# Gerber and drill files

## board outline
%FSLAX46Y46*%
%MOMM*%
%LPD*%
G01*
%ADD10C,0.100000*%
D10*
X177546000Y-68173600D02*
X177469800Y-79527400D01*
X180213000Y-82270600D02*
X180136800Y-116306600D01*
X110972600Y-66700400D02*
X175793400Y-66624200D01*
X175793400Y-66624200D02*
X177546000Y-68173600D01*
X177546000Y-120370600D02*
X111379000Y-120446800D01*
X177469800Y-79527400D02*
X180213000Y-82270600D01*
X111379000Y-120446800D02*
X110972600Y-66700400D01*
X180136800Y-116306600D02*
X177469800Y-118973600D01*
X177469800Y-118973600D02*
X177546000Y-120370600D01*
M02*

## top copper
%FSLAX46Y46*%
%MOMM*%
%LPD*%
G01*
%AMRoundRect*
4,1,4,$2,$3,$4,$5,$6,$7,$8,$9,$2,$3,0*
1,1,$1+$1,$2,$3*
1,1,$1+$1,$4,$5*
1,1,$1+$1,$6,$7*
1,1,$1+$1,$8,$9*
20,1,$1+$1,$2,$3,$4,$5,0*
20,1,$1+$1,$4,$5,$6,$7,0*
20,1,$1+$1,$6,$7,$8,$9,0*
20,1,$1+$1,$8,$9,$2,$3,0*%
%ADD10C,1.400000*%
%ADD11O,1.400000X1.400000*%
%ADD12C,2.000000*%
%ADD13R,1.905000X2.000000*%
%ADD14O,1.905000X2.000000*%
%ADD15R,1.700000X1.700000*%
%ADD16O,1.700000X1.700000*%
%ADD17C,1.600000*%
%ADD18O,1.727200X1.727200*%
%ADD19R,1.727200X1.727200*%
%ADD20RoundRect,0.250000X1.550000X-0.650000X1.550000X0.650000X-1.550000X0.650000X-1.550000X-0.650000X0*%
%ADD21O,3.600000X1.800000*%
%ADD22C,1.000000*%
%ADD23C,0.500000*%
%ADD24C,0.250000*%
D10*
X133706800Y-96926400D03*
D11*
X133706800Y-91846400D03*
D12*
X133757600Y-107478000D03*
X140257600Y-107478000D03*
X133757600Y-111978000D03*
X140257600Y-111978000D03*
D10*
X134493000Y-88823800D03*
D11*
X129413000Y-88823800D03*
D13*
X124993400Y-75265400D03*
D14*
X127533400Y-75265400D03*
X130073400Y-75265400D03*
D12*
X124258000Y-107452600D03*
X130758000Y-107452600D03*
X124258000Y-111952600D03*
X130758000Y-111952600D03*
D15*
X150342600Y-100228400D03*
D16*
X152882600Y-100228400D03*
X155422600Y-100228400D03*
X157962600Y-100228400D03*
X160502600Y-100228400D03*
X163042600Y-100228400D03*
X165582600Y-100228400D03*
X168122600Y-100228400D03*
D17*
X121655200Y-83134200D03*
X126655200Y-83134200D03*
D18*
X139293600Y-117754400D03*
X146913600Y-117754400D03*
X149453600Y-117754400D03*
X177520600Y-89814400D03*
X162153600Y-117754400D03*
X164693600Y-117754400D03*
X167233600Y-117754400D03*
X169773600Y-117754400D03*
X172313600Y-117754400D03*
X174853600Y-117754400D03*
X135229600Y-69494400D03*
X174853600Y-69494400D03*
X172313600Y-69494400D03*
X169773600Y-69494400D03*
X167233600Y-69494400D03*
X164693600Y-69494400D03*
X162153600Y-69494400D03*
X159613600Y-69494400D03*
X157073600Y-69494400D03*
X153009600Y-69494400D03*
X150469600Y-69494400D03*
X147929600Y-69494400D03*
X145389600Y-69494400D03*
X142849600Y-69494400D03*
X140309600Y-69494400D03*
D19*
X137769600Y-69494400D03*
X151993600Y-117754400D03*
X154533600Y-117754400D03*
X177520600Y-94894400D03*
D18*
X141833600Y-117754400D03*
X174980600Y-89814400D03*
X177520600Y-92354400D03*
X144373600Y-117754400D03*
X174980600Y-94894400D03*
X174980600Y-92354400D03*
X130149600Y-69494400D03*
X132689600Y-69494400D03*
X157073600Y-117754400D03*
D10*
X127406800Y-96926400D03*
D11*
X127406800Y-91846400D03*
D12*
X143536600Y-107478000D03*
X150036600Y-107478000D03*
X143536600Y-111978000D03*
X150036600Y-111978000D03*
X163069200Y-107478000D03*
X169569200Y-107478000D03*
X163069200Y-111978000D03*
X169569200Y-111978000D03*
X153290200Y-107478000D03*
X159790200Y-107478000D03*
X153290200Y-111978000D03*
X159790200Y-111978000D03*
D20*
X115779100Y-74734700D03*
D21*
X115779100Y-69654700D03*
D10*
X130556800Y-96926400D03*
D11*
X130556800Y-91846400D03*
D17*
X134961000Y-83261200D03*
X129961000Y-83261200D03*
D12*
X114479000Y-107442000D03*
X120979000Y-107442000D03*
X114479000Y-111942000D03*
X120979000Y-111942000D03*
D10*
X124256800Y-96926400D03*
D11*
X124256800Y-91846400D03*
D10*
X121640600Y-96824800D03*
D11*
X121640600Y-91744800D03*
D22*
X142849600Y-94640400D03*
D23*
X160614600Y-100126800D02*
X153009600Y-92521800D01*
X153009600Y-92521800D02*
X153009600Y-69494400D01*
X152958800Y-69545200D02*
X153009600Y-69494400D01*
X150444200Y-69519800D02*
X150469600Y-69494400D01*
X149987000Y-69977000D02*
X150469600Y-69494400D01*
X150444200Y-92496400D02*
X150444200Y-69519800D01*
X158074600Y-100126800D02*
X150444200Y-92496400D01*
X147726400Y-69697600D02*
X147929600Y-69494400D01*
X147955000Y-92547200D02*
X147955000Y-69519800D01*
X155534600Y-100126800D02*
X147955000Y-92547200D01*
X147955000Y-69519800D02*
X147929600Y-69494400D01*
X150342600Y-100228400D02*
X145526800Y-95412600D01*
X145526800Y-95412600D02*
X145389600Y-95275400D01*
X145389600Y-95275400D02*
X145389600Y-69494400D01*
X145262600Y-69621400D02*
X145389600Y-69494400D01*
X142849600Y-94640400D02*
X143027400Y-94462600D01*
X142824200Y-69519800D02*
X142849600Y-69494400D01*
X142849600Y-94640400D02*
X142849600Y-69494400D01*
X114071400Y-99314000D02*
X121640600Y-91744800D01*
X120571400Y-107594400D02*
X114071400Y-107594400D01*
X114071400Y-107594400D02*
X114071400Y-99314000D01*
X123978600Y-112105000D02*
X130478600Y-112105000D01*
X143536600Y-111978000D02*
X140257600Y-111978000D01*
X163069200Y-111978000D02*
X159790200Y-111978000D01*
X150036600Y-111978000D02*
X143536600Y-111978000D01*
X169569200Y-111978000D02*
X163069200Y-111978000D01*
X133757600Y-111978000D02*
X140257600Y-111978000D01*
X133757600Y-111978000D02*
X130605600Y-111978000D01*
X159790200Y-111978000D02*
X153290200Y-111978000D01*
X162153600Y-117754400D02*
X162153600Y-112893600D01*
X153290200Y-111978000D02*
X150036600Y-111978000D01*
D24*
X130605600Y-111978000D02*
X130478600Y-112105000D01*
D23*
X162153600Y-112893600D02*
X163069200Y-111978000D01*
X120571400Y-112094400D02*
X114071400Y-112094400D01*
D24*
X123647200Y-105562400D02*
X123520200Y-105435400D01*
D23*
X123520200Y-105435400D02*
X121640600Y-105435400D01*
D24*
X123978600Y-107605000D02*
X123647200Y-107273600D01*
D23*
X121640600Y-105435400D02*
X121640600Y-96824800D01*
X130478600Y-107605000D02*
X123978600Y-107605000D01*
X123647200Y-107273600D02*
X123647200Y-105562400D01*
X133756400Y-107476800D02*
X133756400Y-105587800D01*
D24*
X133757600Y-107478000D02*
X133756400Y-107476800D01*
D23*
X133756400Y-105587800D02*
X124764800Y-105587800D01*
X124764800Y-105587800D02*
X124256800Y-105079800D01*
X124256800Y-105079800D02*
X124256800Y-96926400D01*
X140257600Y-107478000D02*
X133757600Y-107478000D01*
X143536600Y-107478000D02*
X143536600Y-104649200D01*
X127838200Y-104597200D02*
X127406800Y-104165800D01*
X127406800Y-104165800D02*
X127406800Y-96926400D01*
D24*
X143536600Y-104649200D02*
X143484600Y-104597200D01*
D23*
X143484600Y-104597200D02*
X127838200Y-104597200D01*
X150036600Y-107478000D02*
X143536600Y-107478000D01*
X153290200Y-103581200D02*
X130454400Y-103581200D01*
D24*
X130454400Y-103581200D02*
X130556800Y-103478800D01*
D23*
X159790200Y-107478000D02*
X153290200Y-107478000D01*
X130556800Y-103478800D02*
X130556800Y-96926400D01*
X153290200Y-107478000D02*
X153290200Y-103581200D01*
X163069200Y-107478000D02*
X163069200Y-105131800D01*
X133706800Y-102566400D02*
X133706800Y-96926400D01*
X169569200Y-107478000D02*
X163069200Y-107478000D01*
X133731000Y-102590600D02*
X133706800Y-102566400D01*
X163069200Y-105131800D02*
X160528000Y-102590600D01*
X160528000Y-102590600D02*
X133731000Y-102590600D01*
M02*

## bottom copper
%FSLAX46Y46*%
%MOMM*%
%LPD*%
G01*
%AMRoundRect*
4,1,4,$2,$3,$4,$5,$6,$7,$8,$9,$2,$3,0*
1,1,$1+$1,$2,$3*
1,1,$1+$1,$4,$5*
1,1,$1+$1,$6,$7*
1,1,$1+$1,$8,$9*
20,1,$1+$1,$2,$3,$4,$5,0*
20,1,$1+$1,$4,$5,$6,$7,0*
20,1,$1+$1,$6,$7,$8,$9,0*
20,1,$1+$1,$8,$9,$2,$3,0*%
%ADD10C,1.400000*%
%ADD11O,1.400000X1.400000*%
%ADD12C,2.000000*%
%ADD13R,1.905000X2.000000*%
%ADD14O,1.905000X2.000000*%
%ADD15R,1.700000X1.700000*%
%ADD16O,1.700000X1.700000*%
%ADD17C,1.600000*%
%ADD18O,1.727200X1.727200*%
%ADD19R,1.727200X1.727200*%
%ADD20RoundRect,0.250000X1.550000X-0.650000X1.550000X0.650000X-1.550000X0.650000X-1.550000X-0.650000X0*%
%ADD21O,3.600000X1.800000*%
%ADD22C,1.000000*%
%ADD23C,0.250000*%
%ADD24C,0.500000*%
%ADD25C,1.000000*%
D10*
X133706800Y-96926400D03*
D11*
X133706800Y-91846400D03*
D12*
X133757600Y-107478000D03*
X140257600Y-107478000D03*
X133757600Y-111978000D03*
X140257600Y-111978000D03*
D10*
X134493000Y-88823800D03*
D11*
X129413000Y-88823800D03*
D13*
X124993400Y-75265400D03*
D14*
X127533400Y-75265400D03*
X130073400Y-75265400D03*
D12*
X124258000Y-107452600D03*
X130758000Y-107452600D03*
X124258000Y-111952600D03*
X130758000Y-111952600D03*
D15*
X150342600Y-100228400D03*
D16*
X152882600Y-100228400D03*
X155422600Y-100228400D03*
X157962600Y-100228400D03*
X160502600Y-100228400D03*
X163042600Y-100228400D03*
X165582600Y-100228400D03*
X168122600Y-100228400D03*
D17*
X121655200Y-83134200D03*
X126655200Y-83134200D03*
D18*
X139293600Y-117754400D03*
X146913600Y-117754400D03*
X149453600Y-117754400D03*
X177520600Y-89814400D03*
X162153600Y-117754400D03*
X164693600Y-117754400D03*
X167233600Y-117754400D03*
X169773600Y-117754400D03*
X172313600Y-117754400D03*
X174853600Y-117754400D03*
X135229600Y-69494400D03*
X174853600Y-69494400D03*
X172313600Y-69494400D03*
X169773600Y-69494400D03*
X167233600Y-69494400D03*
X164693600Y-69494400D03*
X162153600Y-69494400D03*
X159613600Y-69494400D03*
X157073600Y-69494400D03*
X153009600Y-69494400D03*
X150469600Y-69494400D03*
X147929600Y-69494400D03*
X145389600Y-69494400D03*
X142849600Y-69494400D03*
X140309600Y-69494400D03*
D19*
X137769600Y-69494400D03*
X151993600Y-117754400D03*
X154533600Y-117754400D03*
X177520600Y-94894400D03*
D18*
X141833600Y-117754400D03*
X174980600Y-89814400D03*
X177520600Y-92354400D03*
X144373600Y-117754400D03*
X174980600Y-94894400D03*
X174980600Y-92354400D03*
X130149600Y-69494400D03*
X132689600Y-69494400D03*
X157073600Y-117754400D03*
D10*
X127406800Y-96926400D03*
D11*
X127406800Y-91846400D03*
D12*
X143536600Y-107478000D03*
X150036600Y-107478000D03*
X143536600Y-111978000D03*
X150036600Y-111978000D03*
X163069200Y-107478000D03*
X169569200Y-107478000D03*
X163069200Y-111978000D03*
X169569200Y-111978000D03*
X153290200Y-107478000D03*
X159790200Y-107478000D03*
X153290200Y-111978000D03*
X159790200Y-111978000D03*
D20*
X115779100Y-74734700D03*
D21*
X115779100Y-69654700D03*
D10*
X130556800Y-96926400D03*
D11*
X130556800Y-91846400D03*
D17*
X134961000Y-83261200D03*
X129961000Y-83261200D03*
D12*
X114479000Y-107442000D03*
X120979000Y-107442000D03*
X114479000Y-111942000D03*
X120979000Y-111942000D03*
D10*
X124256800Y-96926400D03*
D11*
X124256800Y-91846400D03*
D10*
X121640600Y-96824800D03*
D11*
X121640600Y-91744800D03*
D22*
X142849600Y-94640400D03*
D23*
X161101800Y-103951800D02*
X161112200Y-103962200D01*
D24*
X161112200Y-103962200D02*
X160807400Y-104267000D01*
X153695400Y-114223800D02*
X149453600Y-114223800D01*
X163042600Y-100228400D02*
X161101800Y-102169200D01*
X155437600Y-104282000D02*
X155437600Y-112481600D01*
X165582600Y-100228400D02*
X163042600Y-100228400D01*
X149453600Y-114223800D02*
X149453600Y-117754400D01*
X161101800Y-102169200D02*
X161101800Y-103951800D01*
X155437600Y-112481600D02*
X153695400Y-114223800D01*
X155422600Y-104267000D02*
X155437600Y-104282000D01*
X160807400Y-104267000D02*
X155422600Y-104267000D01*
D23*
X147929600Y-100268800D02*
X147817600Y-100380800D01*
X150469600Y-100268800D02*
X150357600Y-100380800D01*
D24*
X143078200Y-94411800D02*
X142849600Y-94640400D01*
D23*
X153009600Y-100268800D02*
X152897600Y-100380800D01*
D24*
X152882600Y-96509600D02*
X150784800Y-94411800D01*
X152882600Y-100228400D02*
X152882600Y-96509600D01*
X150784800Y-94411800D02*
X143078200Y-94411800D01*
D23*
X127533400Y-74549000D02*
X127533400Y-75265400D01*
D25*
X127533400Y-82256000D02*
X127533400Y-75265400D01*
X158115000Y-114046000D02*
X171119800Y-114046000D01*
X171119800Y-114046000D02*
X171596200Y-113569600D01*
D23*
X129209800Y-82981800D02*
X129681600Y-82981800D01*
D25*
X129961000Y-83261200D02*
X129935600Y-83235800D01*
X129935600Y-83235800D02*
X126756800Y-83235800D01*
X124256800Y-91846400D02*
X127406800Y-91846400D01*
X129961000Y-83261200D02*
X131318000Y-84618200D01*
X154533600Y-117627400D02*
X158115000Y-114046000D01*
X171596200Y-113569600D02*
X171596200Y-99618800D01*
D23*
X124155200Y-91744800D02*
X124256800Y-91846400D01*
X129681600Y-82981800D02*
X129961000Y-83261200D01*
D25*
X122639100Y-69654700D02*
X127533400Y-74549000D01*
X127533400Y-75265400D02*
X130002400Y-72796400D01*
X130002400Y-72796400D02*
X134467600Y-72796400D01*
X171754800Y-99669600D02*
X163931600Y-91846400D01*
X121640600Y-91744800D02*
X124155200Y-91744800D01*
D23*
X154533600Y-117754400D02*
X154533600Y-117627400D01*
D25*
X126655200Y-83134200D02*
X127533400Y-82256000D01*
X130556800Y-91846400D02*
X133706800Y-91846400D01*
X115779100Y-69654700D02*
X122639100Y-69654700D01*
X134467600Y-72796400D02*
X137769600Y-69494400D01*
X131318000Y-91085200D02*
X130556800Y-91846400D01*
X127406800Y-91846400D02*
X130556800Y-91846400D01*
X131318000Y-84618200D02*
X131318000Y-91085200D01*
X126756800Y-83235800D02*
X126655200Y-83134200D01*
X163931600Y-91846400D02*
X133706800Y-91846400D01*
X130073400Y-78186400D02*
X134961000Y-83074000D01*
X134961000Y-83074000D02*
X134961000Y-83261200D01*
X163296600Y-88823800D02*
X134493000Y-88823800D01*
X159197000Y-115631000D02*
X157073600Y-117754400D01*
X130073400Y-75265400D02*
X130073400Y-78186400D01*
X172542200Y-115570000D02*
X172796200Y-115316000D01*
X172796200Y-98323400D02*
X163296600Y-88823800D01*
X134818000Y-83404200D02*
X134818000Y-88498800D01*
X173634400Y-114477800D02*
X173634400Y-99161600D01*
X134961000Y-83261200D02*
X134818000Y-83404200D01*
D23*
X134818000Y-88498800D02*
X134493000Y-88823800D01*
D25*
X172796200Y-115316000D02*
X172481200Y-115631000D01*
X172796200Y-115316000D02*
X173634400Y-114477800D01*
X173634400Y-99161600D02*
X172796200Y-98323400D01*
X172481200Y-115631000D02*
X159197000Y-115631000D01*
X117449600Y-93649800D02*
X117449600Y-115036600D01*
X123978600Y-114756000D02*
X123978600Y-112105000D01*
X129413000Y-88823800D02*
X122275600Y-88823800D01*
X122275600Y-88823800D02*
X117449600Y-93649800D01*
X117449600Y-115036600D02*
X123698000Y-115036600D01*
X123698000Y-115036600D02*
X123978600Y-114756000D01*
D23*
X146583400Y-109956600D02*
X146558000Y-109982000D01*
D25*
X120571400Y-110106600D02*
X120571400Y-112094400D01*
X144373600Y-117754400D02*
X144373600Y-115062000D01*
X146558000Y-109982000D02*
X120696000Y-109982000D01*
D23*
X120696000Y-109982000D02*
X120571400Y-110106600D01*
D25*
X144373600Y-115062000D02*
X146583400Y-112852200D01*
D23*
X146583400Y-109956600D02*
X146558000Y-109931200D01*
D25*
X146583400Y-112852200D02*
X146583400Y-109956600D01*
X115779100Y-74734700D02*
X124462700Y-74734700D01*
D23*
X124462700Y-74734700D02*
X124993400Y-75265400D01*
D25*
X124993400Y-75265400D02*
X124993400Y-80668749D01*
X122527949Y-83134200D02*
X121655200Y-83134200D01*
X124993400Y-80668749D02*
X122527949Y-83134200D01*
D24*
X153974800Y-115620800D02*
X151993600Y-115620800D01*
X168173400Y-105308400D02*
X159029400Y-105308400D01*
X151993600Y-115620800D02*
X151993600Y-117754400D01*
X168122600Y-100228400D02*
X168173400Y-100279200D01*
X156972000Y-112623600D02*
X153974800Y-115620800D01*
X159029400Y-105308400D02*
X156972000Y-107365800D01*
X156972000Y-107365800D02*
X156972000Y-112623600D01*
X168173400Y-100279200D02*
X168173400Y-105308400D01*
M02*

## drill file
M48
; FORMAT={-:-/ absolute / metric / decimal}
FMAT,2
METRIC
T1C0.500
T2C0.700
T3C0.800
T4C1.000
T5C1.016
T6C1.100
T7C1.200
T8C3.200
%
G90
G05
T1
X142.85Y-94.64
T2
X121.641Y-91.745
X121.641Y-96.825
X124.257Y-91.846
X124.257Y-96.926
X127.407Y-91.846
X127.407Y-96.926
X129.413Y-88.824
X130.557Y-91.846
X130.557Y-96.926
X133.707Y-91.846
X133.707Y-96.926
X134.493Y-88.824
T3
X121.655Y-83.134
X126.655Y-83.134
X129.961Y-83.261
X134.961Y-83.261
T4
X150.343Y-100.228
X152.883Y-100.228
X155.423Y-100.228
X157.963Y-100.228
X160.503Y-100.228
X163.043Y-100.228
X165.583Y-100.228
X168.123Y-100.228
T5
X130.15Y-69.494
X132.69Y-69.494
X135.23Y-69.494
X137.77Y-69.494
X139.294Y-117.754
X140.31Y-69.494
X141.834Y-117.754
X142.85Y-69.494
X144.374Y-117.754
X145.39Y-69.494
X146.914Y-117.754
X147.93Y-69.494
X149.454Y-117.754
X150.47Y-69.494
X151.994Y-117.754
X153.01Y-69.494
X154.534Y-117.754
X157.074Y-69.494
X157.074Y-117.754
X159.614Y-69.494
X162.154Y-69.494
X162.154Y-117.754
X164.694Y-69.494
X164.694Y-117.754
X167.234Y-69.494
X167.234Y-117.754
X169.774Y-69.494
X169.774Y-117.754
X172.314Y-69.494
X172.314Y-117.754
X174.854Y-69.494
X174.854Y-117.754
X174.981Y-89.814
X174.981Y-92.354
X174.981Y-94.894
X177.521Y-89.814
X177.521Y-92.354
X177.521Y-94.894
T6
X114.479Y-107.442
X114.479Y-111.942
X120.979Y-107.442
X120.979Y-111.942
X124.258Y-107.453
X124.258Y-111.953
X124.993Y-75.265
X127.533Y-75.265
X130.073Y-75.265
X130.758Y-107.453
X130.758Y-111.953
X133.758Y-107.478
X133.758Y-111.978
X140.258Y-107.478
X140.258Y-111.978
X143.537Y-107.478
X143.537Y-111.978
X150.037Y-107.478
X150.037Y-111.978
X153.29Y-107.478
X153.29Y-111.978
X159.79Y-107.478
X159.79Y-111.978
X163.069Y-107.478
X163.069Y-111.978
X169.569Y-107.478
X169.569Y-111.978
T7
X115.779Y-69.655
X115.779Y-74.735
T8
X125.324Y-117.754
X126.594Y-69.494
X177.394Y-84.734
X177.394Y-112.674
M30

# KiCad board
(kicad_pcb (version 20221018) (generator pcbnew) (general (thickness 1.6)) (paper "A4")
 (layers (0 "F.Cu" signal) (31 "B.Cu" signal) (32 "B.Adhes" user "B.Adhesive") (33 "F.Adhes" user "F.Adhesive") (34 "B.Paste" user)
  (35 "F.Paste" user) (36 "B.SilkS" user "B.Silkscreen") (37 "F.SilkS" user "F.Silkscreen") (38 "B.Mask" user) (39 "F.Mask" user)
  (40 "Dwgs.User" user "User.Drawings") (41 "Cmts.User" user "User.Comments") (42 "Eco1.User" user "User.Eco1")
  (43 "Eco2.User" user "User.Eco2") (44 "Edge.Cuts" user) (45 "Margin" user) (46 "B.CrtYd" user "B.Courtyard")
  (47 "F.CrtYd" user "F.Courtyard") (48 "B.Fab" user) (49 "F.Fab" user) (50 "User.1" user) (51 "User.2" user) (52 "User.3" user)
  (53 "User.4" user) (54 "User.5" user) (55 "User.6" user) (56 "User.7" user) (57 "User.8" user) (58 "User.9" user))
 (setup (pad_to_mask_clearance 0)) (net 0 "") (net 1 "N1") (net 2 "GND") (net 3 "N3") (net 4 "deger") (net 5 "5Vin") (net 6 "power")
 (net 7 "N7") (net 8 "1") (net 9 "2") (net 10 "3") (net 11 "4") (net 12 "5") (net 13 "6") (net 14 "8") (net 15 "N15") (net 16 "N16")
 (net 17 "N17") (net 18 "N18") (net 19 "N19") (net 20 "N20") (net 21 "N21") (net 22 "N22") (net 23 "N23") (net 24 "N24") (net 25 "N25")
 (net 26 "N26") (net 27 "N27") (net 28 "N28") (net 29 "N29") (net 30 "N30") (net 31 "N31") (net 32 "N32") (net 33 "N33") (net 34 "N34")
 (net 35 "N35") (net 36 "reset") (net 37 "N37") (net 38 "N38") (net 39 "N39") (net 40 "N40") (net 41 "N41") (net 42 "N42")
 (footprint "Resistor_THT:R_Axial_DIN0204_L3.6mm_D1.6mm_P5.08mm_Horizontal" (layer "F.Cu") (at 133.7068 96.9264 90)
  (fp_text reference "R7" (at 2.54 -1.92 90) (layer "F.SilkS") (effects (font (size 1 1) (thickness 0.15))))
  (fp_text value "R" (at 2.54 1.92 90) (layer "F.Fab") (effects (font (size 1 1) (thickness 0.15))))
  (pad "1" thru_hole circle (at 0 0 90) (size 1.4 1.4) (drill 0.7) (layers "*.Cu" "*.Mask") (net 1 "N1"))
  (pad "2" thru_hole oval (at 5.08 0 90) (size 1.4 1.4) (drill 0.7) (layers "*.Cu" "*.Mask") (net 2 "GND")))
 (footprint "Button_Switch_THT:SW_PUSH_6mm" (layer "F.Cu") (at 133.7576 107.478)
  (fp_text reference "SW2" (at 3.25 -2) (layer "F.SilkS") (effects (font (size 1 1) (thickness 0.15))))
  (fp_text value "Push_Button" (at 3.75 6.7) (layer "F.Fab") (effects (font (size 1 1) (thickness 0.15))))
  (pad "1" thru_hole circle (at 0 0 90) (size 2 2) (drill 1.1) (layers "*.Cu" "*.Mask") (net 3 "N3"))
  (pad "1" thru_hole circle (at 6.5 0 90) (size 2 2) (drill 1.1) (layers "*.Cu" "*.Mask") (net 3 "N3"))
  (pad "2" thru_hole circle (at 0 4.5 90) (size 2 2) (drill 1.1) (layers "*.Cu" "*.Mask") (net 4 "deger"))
  (pad "2" thru_hole circle (at 6.5 4.5 90) (size 2 2) (drill 1.1) (layers "*.Cu" "*.Mask") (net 4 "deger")))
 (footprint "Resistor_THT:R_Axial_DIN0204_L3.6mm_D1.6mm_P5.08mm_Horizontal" (layer "F.Cu") (at 134.493 88.8238 180)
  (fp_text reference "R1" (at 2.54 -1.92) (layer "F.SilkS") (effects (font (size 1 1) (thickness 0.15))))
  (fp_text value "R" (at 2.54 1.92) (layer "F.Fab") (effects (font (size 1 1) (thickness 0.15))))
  (pad "1" thru_hole circle (at 0 0 180) (size 1.4 1.4) (drill 0.7) (layers "*.Cu" "*.Mask") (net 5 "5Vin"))
  (pad "2" thru_hole oval (at 5.08 0 180) (size 1.4 1.4) (drill 0.7) (layers "*.Cu" "*.Mask") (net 4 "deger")))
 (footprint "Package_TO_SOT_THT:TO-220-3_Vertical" (layer "F.Cu") (at 124.9934 75.2654)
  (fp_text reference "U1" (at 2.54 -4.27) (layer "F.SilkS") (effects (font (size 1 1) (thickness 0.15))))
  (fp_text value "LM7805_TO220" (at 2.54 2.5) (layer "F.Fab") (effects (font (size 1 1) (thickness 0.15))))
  (pad "1" thru_hole rect (at 0 0) (size 1.905 2) (drill 1.1) (layers "*.Cu" "*.Mask") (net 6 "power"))
  (pad "2" thru_hole oval (at 2.54 0) (size 1.905 2) (drill 1.1) (layers "*.Cu" "*.Mask") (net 2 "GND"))
  (pad "3" thru_hole oval (at 5.08 0) (size 1.905 2) (drill 1.1) (layers "*.Cu" "*.Mask") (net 5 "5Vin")))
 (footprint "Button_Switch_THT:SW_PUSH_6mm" (layer "F.Cu") (at 124.258 107.4526)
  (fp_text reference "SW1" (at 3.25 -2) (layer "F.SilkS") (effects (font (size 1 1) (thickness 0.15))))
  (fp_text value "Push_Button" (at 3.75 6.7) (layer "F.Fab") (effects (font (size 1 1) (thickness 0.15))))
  (pad "1" thru_hole circle (at 0 0 90) (size 2 2) (drill 1.1) (layers "*.Cu" "*.Mask") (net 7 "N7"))
  (pad "1" thru_hole circle (at 6.5 0 90) (size 2 2) (drill 1.1) (layers "*.Cu" "*.Mask") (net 7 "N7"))
  (pad "2" thru_hole circle (at 0 4.5 90) (size 2 2) (drill 1.1) (layers "*.Cu" "*.Mask") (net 4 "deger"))
  (pad "2" thru_hole circle (at 6.5 4.5 90) (size 2 2) (drill 1.1) (layers "*.Cu" "*.Mask") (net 4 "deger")))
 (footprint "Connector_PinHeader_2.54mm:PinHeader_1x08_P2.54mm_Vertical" (layer "F.Cu") (at 150.3426 100.2284 90)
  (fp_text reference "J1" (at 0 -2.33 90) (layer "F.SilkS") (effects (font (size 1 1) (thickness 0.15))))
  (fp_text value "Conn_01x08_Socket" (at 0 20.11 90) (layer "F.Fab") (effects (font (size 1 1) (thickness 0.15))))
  (pad "1" thru_hole rect (at 0 0 90) (size 1.7 1.7) (drill 1) (layers "*.Cu" "*.Mask") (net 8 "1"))
  (pad "2" thru_hole oval (at 0 2.54 90) (size 1.7 1.7) (drill 1) (layers "*.Cu" "*.Mask") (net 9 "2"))
  (pad "3" thru_hole oval (at 0 5.08 90) (size 1.7 1.7) (drill 1) (layers "*.Cu" "*.Mask") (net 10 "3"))
  (pad "4" thru_hole oval (at 0 7.62 90) (size 1.7 1.7) (drill 1) (layers "*.Cu" "*.Mask") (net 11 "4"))
  (pad "5" thru_hole oval (at 0 10.16 90) (size 1.7 1.7) (drill 1) (layers "*.Cu" "*.Mask") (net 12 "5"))
  (pad "6" thru_hole oval (at 0 12.7 90) (size 1.7 1.7) (drill 1) (layers "*.Cu" "*.Mask") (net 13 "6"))
  (pad "7" thru_hole oval (at 0 15.24 90) (size 1.7 1.7) (drill 1) (layers "*.Cu" "*.Mask") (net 13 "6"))
  (pad "8" thru_hole oval (at 0 17.78 90) (size 1.7 1.7) (drill 1) (layers "*.Cu" "*.Mask") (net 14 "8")))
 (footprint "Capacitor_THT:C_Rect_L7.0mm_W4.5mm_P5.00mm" (layer "F.Cu") (at 121.6552 83.1342)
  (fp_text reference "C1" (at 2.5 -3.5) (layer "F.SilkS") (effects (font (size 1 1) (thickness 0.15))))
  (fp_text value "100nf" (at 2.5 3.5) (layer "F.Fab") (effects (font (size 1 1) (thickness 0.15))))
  (pad "1" thru_hole circle (at 0 0) (size 1.6 1.6) (drill 0.8) (layers "*.Cu" "*.Mask") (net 6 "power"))
  (pad "2" thru_hole circle (at 5 0) (size 1.6 1.6) (drill 0.8) (layers "*.Cu" "*.Mask") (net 2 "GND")))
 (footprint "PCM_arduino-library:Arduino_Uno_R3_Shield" (layer "F.Cu") (at 111.3536 120.2944)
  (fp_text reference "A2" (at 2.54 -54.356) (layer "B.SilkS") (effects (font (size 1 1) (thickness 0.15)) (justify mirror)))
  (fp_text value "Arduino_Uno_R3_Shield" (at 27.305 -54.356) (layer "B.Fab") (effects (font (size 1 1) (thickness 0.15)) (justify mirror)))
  (pad "" np_thru_hole circle (at 13.97 -2.54) (size 3.2 3.2) (drill 3.2) (layers "*.Cu" "*.Mask"))
  (pad "" np_thru_hole circle (at 15.24 -50.8) (size 3.2 3.2) (drill 3.2) (layers "*.Cu" "*.Mask"))
  (pad "" thru_hole oval (at 27.94 -2.54) (size 1.7272 1.7272) (drill 1.016) (layers "*.Cu" "*.Mask"))
  (pad "" np_thru_hole circle (at 66.04 -35.56) (size 3.2 3.2) (drill 3.2) (layers "*.Cu" "*.Mask"))
  (pad "" np_thru_hole circle (at 66.04 -7.62) (size 3.2 3.2) (drill 3.2) (layers "*.Cu" "*.Mask"))
  (pad "3V3" thru_hole oval (at 35.56 -2.54) (size 1.7272 1.7272) (drill 1.016) (layers "*.Cu" "*.Mask") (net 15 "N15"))
  (pad "5V1" thru_hole oval (at 38.1 -2.54) (size 1.7272 1.7272) (drill 1.016) (layers "*.Cu" "*.Mask") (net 13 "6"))
  (pad "5V2" thru_hole oval (at 66.167 -30.48) (size 1.7272 1.7272) (drill 1.016) (layers "*.Cu" "*.Mask") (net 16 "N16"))
  (pad "A0" thru_hole oval (at 50.8 -2.54) (size 1.7272 1.7272) (drill 1.016) (layers "*.Cu" "*.Mask") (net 4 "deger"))
  (pad "A1" thru_hole oval (at 53.34 -2.54) (size 1.7272 1.7272) (drill 1.016) (layers "*.Cu" "*.Mask") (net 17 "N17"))
  (pad "A2" thru_hole oval (at 55.88 -2.54) (size 1.7272 1.7272) (drill 1.016) (layers "*.Cu" "*.Mask") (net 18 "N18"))
  (pad "A3" thru_hole oval (at 58.42 -2.54) (size 1.7272 1.7272) (drill 1.016) (layers "*.Cu" "*.Mask") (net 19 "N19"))
  (pad "A4" thru_hole oval (at 60.96 -2.54) (size 1.7272 1.7272) (drill 1.016) (layers "*.Cu" "*.Mask") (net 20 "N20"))
  (pad "A5" thru_hole oval (at 63.5 -2.54) (size 1.7272 1.7272) (drill 1.016) (layers "*.Cu" "*.Mask") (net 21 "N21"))
  (pad "AREF" thru_hole oval (at 23.876 -50.8) (size 1.7272 1.7272) (drill 1.016) (layers "*.Cu" "*.Mask") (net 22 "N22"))
  (pad "D0" thru_hole oval (at 63.5 -50.8) (size 1.7272 1.7272) (drill 1.016) (layers "*.Cu" "*.Mask") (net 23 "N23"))
  (pad "D1" thru_hole oval (at 60.96 -50.8) (size 1.7272 1.7272) (drill 1.016) (layers "*.Cu" "*.Mask") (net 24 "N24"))
  (pad "D2" thru_hole oval (at 58.42 -50.8) (size 1.7272 1.7272) (drill 1.016) (layers "*.Cu" "*.Mask") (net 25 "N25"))
  (pad "D3" thru_hole oval (at 55.88 -50.8) (size 1.7272 1.7272) (drill 1.016) (layers "*.Cu" "*.Mask") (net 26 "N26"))
  (pad "D4" thru_hole oval (at 53.34 -50.8) (size 1.7272 1.7272) (drill 1.016) (layers "*.Cu" "*.Mask") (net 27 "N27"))
  (pad "D5" thru_hole oval (at 50.8 -50.8) (size 1.7272 1.7272) (drill 1.016) (layers "*.Cu" "*.Mask") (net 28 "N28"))
  (pad "D6" thru_hole oval (at 48.26 -50.8) (size 1.7272 1.7272) (drill 1.016) (layers "*.Cu" "*.Mask") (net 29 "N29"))
  (pad "D7" thru_hole oval (at 45.72 -50.8) (size 1.7272 1.7272) (drill 1.016) (layers "*.Cu" "*.Mask") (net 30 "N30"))
  (pad "D8" thru_hole oval (at 41.656 -50.8) (size 1.7272 1.7272) (drill 1.016) (layers "*.Cu" "*.Mask") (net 12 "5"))
  (pad "D9" thru_hole oval (at 39.116 -50.8) (size 1.7272 1.7272) (drill 1.016) (layers "*.Cu" "*.Mask") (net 11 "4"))
  (pad "D10" thru_hole oval (at 36.576 -50.8) (size 1.7272 1.7272) (drill 1.016) (layers "*.Cu" "*.Mask") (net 10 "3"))
  (pad "D11" thru_hole oval (at 34.036 -50.8) (size 1.7272 1.7272) (drill 1.016) (layers "*.Cu" "*.Mask") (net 8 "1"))
  (pad "D12" thru_hole oval (at 31.496 -50.8) (size 1.7272 1.7272) (drill 1.016) (layers "*.Cu" "*.Mask") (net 9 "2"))
  (pad "D13" thru_hole oval (at 28.956 -50.8) (size 1.7272 1.7272) (drill 1.016) (layers "*.Cu" "*.Mask") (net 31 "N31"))
  (pad "GND1" thru_hole rect (at 26.416 -50.8) (size 1.7272 1.7272) (drill 1.016) (layers "*.Cu" "*.Mask") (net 2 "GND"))
  (pad "GND2" thru_hole rect (at 40.64 -2.54) (size 1.7272 1.7272) (drill 1.016) (layers "*.Cu" "*.Mask") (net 14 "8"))
  (pad "GND3" thru_hole rect (at 43.18 -2.54) (size 1.7272 1.7272) (drill 1.016) (layers "*.Cu" "*.Mask") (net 2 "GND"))
  (pad "GND4" thru_hole rect (at 66.167 -25.4) (size 1.7272 1.7272) (drill 1.016) (layers "*.Cu" "*.Mask") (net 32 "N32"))
  (pad "IORF" thru_hole oval (at 30.48 -2.54) (size 1.7272 1.7272) (drill 1.016) (layers "*.Cu" "*.Mask") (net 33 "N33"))
  (pad "MISO" thru_hole oval (at 63.627 -30.48) (size 1.7272 1.7272) (drill 1.016) (layers "*.Cu" "*.Mask") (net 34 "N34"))
  (pad "MOSI" thru_hole oval (at 66.167 -27.94) (size 1.7272 1.7272) (drill 1.016) (layers "*.Cu" "*.Mask") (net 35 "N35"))
  (pad "RST1" thru_hole oval (at 33.02 -2.54) (size 1.7272 1.7272) (drill 1.016) (layers "*.Cu" "*.Mask") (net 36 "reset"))
  (pad "RST2" thru_hole oval (at 63.627 -25.4) (size 1.7272 1.7272) (drill 1.016) (layers "*.Cu" "*.Mask") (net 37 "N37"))
  (pad "SCK" thru_hole oval (at 63.627 -27.94) (size 1.7272 1.7272) (drill 1.016) (layers "*.Cu" "*.Mask") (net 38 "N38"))
  (pad "SCL" thru_hole oval (at 18.796 -50.8) (size 1.7272 1.7272) (drill 1.016) (layers "*.Cu" "*.Mask") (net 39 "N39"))
  (pad "SDA" thru_hole oval (at 21.336 -50.8) (size 1.7272 1.7272) (drill 1.016) (layers "*.Cu" "*.Mask") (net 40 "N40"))
  (pad "VIN" thru_hole oval (at 45.72 -2.54) (size 1.7272 1.7272) (drill 1.016) (layers "*.Cu" "*.Mask") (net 5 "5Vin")))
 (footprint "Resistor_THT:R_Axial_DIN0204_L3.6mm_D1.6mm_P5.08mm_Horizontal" (layer "F.Cu") (at 127.4068 96.9264 90)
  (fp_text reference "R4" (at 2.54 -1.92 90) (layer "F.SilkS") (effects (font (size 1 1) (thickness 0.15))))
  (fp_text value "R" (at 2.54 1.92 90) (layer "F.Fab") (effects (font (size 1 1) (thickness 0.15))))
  (pad "1" thru_hole circle (at 0 0 90) (size 1.4 1.4) (drill 0.7) (layers "*.Cu" "*.Mask") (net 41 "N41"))
  (pad "2" thru_hole oval (at 5.08 0 90) (size 1.4 1.4) (drill 0.7) (layers "*.Cu" "*.Mask") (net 2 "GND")))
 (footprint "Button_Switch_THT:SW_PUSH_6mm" (layer "F.Cu") (at 143.5366 107.478)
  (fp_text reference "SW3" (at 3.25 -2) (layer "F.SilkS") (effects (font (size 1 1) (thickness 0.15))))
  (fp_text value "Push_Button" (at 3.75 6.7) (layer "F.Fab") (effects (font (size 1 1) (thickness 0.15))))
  (pad "1" thru_hole circle (at 0 0 90) (size 2 2) (drill 1.1) (layers "*.Cu" "*.Mask") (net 41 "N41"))
  (pad "1" thru_hole circle (at 6.5 0 90) (size 2 2) (drill 1.1) (layers "*.Cu" "*.Mask") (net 41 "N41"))
  (pad "2" thru_hole circle (at 0 4.5 90) (size 2 2) (drill 1.1) (layers "*.Cu" "*.Mask") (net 4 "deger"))
  (pad "2" thru_hole circle (at 6.5 4.5 90) (size 2 2) (drill 1.1) (layers "*.Cu" "*.Mask") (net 4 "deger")))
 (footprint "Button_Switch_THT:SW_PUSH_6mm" (layer "F.Cu") (at 163.0692 107.478)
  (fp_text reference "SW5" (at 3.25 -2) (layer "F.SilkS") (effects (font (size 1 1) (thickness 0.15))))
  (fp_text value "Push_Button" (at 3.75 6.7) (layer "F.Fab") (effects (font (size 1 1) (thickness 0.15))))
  (pad "1" thru_hole circle (at 0 0 90) (size 2 2) (drill 1.1) (layers "*.Cu" "*.Mask") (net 1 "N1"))
  (pad "1" thru_hole circle (at 6.5 0 90) (size 2 2) (drill 1.1) (layers "*.Cu" "*.Mask") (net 1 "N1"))
  (pad "2" thru_hole circle (at 0 4.5 90) (size 2 2) (drill 1.1) (layers "*.Cu" "*.Mask") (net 4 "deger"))
  (pad "2" thru_hole circle (at 6.5 4.5 90) (size 2 2) (drill 1.1) (layers "*.Cu" "*.Mask") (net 4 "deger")))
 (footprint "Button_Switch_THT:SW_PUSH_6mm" (layer "F.Cu") (at 153.2902 107.478)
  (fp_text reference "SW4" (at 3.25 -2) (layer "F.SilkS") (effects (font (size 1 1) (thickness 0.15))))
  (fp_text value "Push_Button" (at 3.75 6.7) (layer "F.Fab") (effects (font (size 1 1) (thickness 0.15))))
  (pad "1" thru_hole circle (at 0 0 90) (size 2 2) (drill 1.1) (layers "*.Cu" "*.Mask") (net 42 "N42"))
  (pad "1" thru_hole circle (at 6.5 0 90) (size 2 2) (drill 1.1) (layers "*.Cu" "*.Mask") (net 42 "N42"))
  (pad "2" thru_hole circle (at 0 4.5 90) (size 2 2) (drill 1.1) (layers "*.Cu" "*.Mask") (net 4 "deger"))
  (pad "2" thru_hole circle (at 6.5 4.5 90) (size 2 2) (drill 1.1) (layers "*.Cu" "*.Mask") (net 4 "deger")))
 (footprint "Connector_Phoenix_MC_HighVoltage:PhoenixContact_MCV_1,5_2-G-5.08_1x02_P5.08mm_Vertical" (layer "F.Cu") (at 115.7791 74.7347 90)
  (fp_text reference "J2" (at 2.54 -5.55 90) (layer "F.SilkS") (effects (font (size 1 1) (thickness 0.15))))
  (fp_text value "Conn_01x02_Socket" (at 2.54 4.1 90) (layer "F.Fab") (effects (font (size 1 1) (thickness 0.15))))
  (pad "1" thru_hole roundrect (at 0 0 90) (size 1.8 3.6) (drill 1.2) (layers "*.Cu" "*.Mask") (roundrect_rratio 0.138889) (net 6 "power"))
  (pad "2" thru_hole oval (at 5.08 0 90) (size 1.8 3.6) (drill 1.2) (layers "*.Cu" "*.Mask") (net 2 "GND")))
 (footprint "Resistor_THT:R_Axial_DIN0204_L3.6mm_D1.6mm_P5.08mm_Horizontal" (layer "F.Cu") (at 130.5568 96.9264 90)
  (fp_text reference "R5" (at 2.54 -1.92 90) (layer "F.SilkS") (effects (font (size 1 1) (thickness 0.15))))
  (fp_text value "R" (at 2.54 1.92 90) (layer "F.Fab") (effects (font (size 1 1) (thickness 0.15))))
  (pad "1" thru_hole circle (at 0 0 90) (size 1.4 1.4) (drill 0.7) (layers "*.Cu" "*.Mask") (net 42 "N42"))
  (pad "2" thru_hole oval (at 5.08 0 90) (size 1.4 1.4) (drill 0.7) (layers "*.Cu" "*.Mask") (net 2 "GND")))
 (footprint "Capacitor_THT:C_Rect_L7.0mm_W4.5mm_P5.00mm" (layer "F.Cu") (at 134.961 83.2612 180)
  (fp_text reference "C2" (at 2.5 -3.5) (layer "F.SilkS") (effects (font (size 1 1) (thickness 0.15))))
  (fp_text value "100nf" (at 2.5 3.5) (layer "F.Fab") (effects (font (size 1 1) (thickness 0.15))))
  (pad "1" thru_hole circle (at 0 0 180) (size 1.6 1.6) (drill 0.8) (layers "*.Cu" "*.Mask") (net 5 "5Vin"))
  (pad "2" thru_hole circle (at 5 0 180) (size 1.6 1.6) (drill 0.8) (layers "*.Cu" "*.Mask") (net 2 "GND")))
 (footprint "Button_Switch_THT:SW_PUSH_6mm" (layer "F.Cu") (at 114.479 107.442)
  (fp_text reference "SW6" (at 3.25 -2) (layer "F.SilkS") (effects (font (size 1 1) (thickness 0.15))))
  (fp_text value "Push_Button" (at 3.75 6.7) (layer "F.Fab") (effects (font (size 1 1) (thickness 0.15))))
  (pad "1" thru_hole circle (at 0 0 90) (size 2 2) (drill 1.1) (layers "*.Cu" "*.Mask") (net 2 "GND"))
  (pad "1" thru_hole circle (at 6.5 0 90) (size 2 2) (drill 1.1) (layers "*.Cu" "*.Mask") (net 2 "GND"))
  (pad "2" thru_hole circle (at 0 4.5 90) (size 2 2) (drill 1.1) (layers "*.Cu" "*.Mask") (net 36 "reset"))
  (pad "2" thru_hole circle (at 6.5 4.5 90) (size 2 2) (drill 1.1) (layers "*.Cu" "*.Mask") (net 36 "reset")))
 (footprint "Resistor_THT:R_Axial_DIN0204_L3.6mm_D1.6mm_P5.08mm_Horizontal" (layer "F.Cu") (at 124.2568 96.9264 90)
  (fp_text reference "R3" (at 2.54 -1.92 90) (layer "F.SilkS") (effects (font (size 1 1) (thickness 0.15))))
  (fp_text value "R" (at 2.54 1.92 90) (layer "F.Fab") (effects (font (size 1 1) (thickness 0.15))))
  (pad "1" thru_hole circle (at 0 0 90) (size 1.4 1.4) (drill 0.7) (layers "*.Cu" "*.Mask") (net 3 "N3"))
  (pad "2" thru_hole oval (at 5.08 0 90) (size 1.4 1.4) (drill 0.7) (layers "*.Cu" "*.Mask") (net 2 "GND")))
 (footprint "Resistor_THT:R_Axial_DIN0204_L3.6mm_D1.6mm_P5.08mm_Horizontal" (layer "F.Cu") (at 121.6406 96.8248 90)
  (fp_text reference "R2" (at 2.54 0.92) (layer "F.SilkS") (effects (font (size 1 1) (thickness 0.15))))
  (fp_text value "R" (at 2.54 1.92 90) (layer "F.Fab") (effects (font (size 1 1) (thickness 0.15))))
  (pad "1" thru_hole circle (at 0 0 90) (size 1.4 1.4) (drill 0.7) (layers "*.Cu" "*.Mask") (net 7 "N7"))
  (pad "2" thru_hole oval (at 5.08 0 90) (size 1.4 1.4) (drill 0.7) (layers "*.Cu" "*.Mask") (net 2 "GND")))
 (gr_line (start 177.546 68.1736) (end 177.4698 79.5274) (stroke (width 0.1) (type default)) (layer "Edge.Cuts"))
 (gr_line (start 180.213 82.2706) (end 180.1368 116.3066) (stroke (width 0.1) (type default)) (layer "Edge.Cuts"))
 (gr_line (start 110.9726 66.7004) (end 175.7934 66.6242) (stroke (width 0.1) (type default)) (layer "Edge.Cuts"))
 (gr_line (start 175.7934 66.6242) (end 177.546 68.1736) (stroke (width 0.1) (type default)) (layer "Edge.Cuts"))
 (gr_line (start 177.546 120.3706) (end 111.379 120.4468) (stroke (width 0.1) (type default)) (layer "Edge.Cuts"))
 (gr_line (start 177.4698 79.5274) (end 180.213 82.2706) (stroke (width 0.1) (type default)) (layer "Edge.Cuts"))
 (gr_line (start 111.379 120.4468) (end 110.9726 66.7004) (stroke (width 0.1) (type default)) (layer "Edge.Cuts"))
 (gr_line (start 180.1368 116.3066) (end 177.4698 118.9736) (stroke (width 0.1) (type default)) (layer "Edge.Cuts"))
 (gr_line (start 177.4698 118.9736) (end 177.546 120.3706) (stroke (width 0.1) (type default)) (layer "Edge.Cuts"))
 (segment (start 161.1018 103.9518) (end 161.1122 103.9622) (width 0.25) (layer "B.Cu") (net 13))
 (segment (start 161.1122 103.9622) (end 160.8074 104.267) (width 0.5) (layer "B.Cu") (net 13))
 (segment (start 153.6954 114.2238) (end 149.4536 114.2238) (width 0.5) (layer "B.Cu") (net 13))
 (segment (start 163.0426 100.2284) (end 161.1018 102.1692) (width 0.5) (layer "B.Cu") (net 13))
 (segment (start 155.4376 104.282) (end 155.4376 112.4816) (width 0.5) (layer "B.Cu") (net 13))
 (segment (start 165.5826 100.2284) (end 163.0426 100.2284) (width 0.5) (layer "B.Cu") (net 13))
 (segment (start 149.4536 114.2238) (end 149.4536 117.7544) (width 0.5) (layer "B.Cu") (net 13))
 (segment (start 161.1018 102.1692) (end 161.1018 103.9518) (width 0.5) (layer "B.Cu") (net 13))
 (segment (start 155.4376 112.4816) (end 153.6954 114.2238) (width 0.5) (layer "B.Cu") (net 13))
 (segment (start 155.4226 104.267) (end 155.4376 104.282) (width 0.5) (layer "B.Cu") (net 13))
 (segment (start 160.8074 104.267) (end 155.4226 104.267) (width 0.5) (layer "B.Cu") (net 13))
 (segment (start 160.6146 100.1268) (end 153.0096 92.5218) (width 0.5) (layer "F.Cu") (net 12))
 (segment (start 153.0096 92.5218) (end 153.0096 69.4944) (width 0.5) (layer "F.Cu") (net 12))
 (segment (start 152.9588 69.5452) (end 153.0096 69.4944) (width 0.5) (layer "F.Cu") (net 12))
 (segment (start 150.4442 69.5198) (end 150.4696 69.4944) (width 0.5) (layer "F.Cu") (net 11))
 (segment (start 149.987 69.977) (end 150.4696 69.4944) (width 0.5) (layer "F.Cu") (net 11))
 (segment (start 150.4442 92.4964) (end 150.4442 69.5198) (width 0.5) (layer "F.Cu") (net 11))
 (segment (start 158.0746 100.1268) (end 150.4442 92.4964) (width 0.5) (layer "F.Cu") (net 11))
 (segment (start 147.7264 69.6976) (end 147.9296 69.4944) (width 0.5) (layer "F.Cu") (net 10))
 (segment (start 147.955 92.5472) (end 147.955 69.5198) (width 0.5) (layer "F.Cu") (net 10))
 (segment (start 155.5346 100.1268) (end 147.955 92.5472) (width 0.5) (layer "F.Cu") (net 10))
 (segment (start 147.955 69.5198) (end 147.9296 69.4944) (width 0.5) (layer "F.Cu") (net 10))
 (segment (start 150.3426 100.2284) (end 145.5268 95.4126) (width 0.5) (layer "F.Cu") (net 8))
 (segment (start 145.5268 95.4126) (end 145.3896 95.2754) (width 0.5) (layer "F.Cu") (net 8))
 (segment (start 145.3896 95.2754) (end 145.3896 69.4944) (width 0.5) (layer "F.Cu") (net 8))
 (segment (start 145.2626 69.6214) (end 145.3896 69.4944) (width 0.5) (layer "F.Cu") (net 8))
 (segment (start 147.9296 100.2688) (end 147.8176 100.3808) (width 0.25) (layer "B.Cu") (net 8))
 (segment (start 150.4696 100.2688) (end 150.3576 100.3808) (width 0.25) (layer "B.Cu") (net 8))
 (segment (start 142.8496 94.6404) (end 143.0274 94.4626) (width 0.5) (layer "F.Cu") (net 9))
 (segment (start 142.8242 69.5198) (end 142.8496 69.4944) (width 0.5) (layer "F.Cu") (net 9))
 (segment (start 142.8496 94.6404) (end 142.8496 69.4944) (width 0.5) (layer "F.Cu") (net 9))
 (via (at 142.8496 94.6404) (size 1) (drill 0.5) (layers "F.Cu" "B.Cu") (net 9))
 (segment (start 143.0782 94.4118) (end 142.8496 94.6404) (width 0.5) (layer "B.Cu") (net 9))
 (segment (start 153.0096 100.2688) (end 152.8976 100.3808) (width 0.25) (layer "B.Cu") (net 9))
 (segment (start 152.8826 96.5096) (end 150.7848 94.4118) (width 0.5) (layer "B.Cu") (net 9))
 (segment (start 152.8826 100.2284) (end 152.8826 96.5096) (width 0.5) (layer "B.Cu") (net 9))
 (segment (start 150.7848 94.4118) (end 143.0782 94.4118) (width 0.5) (layer "B.Cu") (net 9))
 (segment (start 114.0714 99.314) (end 121.6406 91.7448) (width 0.5) (layer "F.Cu") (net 2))
 (segment (start 120.5714 107.5944) (end 114.0714 107.5944) (width 0.5) (layer "F.Cu") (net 2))
 (segment (start 114.0714 107.5944) (end 114.0714 99.314) (width 0.5) (layer "F.Cu") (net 2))
 (segment (start 127.5334 74.549) (end 127.5334 75.2654) (width 0.25) (layer "B.Cu") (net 2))
 (segment (start 127.5334 82.256) (end 127.5334 75.2654) (width 1) (layer "B.Cu") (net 2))
 (segment (start 158.115 114.046) (end 171.1198 114.046) (width 1) (layer "B.Cu") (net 2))
 (segment (start 171.1198 114.046) (end 171.5962 113.5696) (width 1) (layer "B.Cu") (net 2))
 (segment (start 129.2098 82.9818) (end 129.6816 82.9818) (width 0.25) (layer "B.Cu") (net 2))
 (segment (start 129.961 83.2612) (end 129.9356 83.2358) (width 1) (layer "B.Cu") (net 2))
 (segment (start 129.9356 83.2358) (end 126.7568 83.2358) (width 1) (layer "B.Cu") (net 2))
 (segment (start 124.2568 91.8464) (end 127.4068 91.8464) (width 1) (layer "B.Cu") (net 2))
 (segment (start 129.961 83.2612) (end 131.318 84.6182) (width 1) (layer "B.Cu") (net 2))
 (segment (start 154.5336 117.6274) (end 158.115 114.046) (width 1) (layer "B.Cu") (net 2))
 (segment (start 171.5962 113.5696) (end 171.5962 99.6188) (width 1) (layer "B.Cu") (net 2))
 (segment (start 124.1552 91.7448) (end 124.2568 91.8464) (width 0.25) (layer "B.Cu") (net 2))
 (segment (start 129.6816 82.9818) (end 129.961 83.2612) (width 0.25) (layer "B.Cu") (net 2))
 (segment (start 122.6391 69.6547) (end 127.5334 74.549) (width 1) (layer "B.Cu") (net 2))
 (segment (start 127.5334 75.2654) (end 130.0024 72.7964) (width 1) (layer "B.Cu") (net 2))
 (segment (start 130.0024 72.7964) (end 134.4676 72.7964) (width 1) (layer "B.Cu") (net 2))
 (segment (start 171.7548 99.6696) (end 163.9316 91.8464) (width 1) (layer "B.Cu") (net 2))
 (segment (start 121.6406 91.7448) (end 124.1552 91.7448) (width 1) (layer "B.Cu") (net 2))
 (segment (start 154.5336 117.7544) (end 154.5336 117.6274) (width 0.25) (layer "B.Cu") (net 2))
 (segment (start 126.6552 83.1342) (end 127.5334 82.256) (width 1) (layer "B.Cu") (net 2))
 (segment (start 130.5568 91.8464) (end 133.7068 91.8464) (width 1) (layer "B.Cu") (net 2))
 (segment (start 115.7791 69.6547) (end 122.6391 69.6547) (width 1) (layer "B.Cu") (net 2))
 (segment (start 134.4676 72.7964) (end 137.7696 69.4944) (width 1) (layer "B.Cu") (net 2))
 (segment (start 131.318 91.0852) (end 130.5568 91.8464) (width 1) (layer "B.Cu") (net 2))
 (segment (start 127.4068 91.8464) (end 130.5568 91.8464) (width 1) (layer "B.Cu") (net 2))
 (segment (start 131.318 84.6182) (end 131.318 91.0852) (width 1) (layer "B.Cu") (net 2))
 (segment (start 126.7568 83.2358) (end 126.6552 83.1342) (width 1) (layer "B.Cu") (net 2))
 (segment (start 163.9316 91.8464) (end 133.7068 91.8464) (width 1) (layer "B.Cu") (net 2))
 (segment (start 130.0734 78.1864) (end 134.961 83.074) (width 1) (layer "B.Cu") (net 5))
 (segment (start 134.961 83.074) (end 134.961 83.2612) (width 1) (layer "B.Cu") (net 5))
 (segment (start 163.2966 88.8238) (end 134.493 88.8238) (width 1) (layer "B.Cu") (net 5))
 (segment (start 159.197 115.631) (end 157.0736 117.7544) (width 1) (layer "B.Cu") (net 5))
 (segment (start 130.0734 75.2654) (end 130.0734 78.1864) (width 1) (layer "B.Cu") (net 5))
 (segment (start 172.5422 115.57) (end 172.7962 115.316) (width 1) (layer "B.Cu") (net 5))
 (segment (start 172.7962 98.3234) (end 163.2966 88.8238) (width 1) (layer "B.Cu") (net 5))
 (segment (start 134.818 83.4042) (end 134.818 88.4988) (width 1) (layer "B.Cu") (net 5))
 (segment (start 173.6344 114.4778) (end 173.6344 99.1616) (width 1) (layer "B.Cu") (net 5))
 (segment (start 134.961 83.2612) (end 134.818 83.4042) (width 1) (layer "B.Cu") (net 5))
 (segment (start 134.818 88.4988) (end 134.493 88.8238) (width 0.25) (layer "B.Cu") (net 5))
 (segment (start 172.7962 115.316) (end 172.4812 115.631) (width 1) (layer "B.Cu") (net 5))
 (segment (start 172.7962 115.316) (end 173.6344 114.4778) (width 1) (layer "B.Cu") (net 5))
 (segment (start 173.6344 99.1616) (end 172.7962 98.3234) (width 1) (layer "B.Cu") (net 5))
 (segment (start 172.4812 115.631) (end 159.197 115.631) (width 1) (layer "B.Cu") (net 5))
 (segment (start 123.9786 112.105) (end 130.4786 112.105) (width 0.5) (layer "F.Cu") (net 4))
 (segment (start 143.5366 111.978) (end 140.2576 111.978) (width 0.5) (layer "F.Cu") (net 4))
 (segment (start 163.0692 111.978) (end 159.7902 111.978) (width 0.5) (layer "F.Cu") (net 4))
 (segment (start 150.0366 111.978) (end 143.5366 111.978) (width 0.5) (layer "F.Cu") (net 4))
 (segment (start 169.5692 111.978) (end 163.0692 111.978) (width 0.5) (layer "F.Cu") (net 4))
 (segment (start 133.7576 111.978) (end 140.2576 111.978) (width 0.5) (layer "F.Cu") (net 4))
 (segment (start 133.7576 111.978) (end 130.6056 111.978) (width 0.5) (layer "F.Cu") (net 4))
 (segment (start 159.7902 111.978) (end 153.2902 111.978) (width 0.5) (layer "F.Cu") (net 4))
 (segment (start 162.1536 117.7544) (end 162.1536 112.8936) (width 0.5) (layer "F.Cu") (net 4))
 (segment (start 153.2902 111.978) (end 150.0366 111.978) (width 0.5) (layer "F.Cu") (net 4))
 (segment (start 130.6056 111.978) (end 130.4786 112.105) (width 0.25) (layer "F.Cu") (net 4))
 (segment (start 162.1536 112.8936) (end 163.0692 111.978) (width 0.5) (layer "F.Cu") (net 4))
 (segment (start 117.4496 93.6498) (end 117.4496 115.0366) (width 1) (layer "B.Cu") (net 4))
 (segment (start 123.9786 114.756) (end 123.9786 112.105) (width 1) (layer "B.Cu") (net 4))
 (segment (start 129.413 88.8238) (end 122.2756 88.8238) (width 1) (layer "B.Cu") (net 4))
 (segment (start 122.2756 88.8238) (end 117.4496 93.6498) (width 1) (layer "B.Cu") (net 4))
 (segment (start 117.4496 115.0366) (end 123.698 115.0366) (width 1) (layer "B.Cu") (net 4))
 (segment (start 123.698 115.0366) (end 123.9786 114.756) (width 1) (layer "B.Cu") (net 4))
 (segment (start 120.5714 112.0944) (end 114.0714 112.0944) (width 0.5) (layer "F.Cu") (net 36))
 (segment (start 146.5834 109.9566) (end 146.558 109.982) (width 0.25) (layer "B.Cu") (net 36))
 (segment (start 120.5714 110.1066) (end 120.5714 112.0944) (width 1) (layer "B.Cu") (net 36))
 (segment (start 144.3736 117.7544) (end 144.3736 115.062) (width 1) (layer "B.Cu") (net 36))
 (segment (start 146.558 109.982) (end 120.696 109.982) (width 1) (layer "B.Cu") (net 36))
 (segment (start 120.696 109.982) (end 120.5714 110.1066) (width 0.25) (layer "B.Cu") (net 36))
 (segment (start 144.3736 115.062) (end 146.5834 112.8522) (width 1) (layer "B.Cu") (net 36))
 (segment (start 146.5834 109.9566) (end 146.558 109.9312) (width 0.25) (layer "B.Cu") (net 36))
 (segment (start 146.5834 112.8522) (end 146.5834 109.9566) (width 1) (layer "B.Cu") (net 36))
 (segment (start 115.7791 74.7347) (end 124.4627 74.7347) (width 1) (layer "B.Cu") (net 6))
 (segment (start 124.4627 74.7347) (end 124.9934 75.2654) (width 0.25) (layer "B.Cu") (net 6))
 (segment (start 124.9934 75.2654) (end 124.9934 80.668749) (width 1) (layer "B.Cu") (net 6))
 (segment (start 122.527949 83.1342) (end 121.6552 83.1342) (width 1) (layer "B.Cu") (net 6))
 (segment (start 124.9934 80.668749) (end 122.527949 83.1342) (width 1) (layer "B.Cu") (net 6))
 (segment (start 123.6472 105.5624) (end 123.5202 105.4354) (width 0.25) (layer "F.Cu") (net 7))
 (segment (start 123.5202 105.4354) (end 121.6406 105.4354) (width 0.5) (layer "F.Cu") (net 7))
 (segment (start 123.9786 107.605) (end 123.6472 107.2736) (width 0.25) (layer "F.Cu") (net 7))
 (segment (start 121.6406 105.4354) (end 121.6406 96.8248) (width 0.5) (layer "F.Cu") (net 7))
 (segment (start 130.4786 107.605) (end 123.9786 107.605) (width 0.5) (layer "F.Cu") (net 7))
 (segment (start 123.6472 107.2736) (end 123.6472 105.5624) (width 0.5) (layer "F.Cu") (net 7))
 (segment (start 133.7564 107.4768) (end 133.7564 105.5878) (width 0.5) (layer "F.Cu") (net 3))
 (segment (start 133.7576 107.478) (end 133.7564 107.4768) (width 0.25) (layer "F.Cu") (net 3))
 (segment (start 133.7564 105.5878) (end 124.7648 105.5878) (width 0.5) (layer "F.Cu") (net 3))
 (segment (start 124.7648 105.5878) (end 124.2568 105.0798) (width 0.5) (layer "F.Cu") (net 3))
 (segment (start 124.2568 105.0798) (end 124.2568 96.9264) (width 0.5) (layer "F.Cu") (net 3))
 (segment (start 140.2576 107.478) (end 133.7576 107.478) (width 0.5) (layer "F.Cu") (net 3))
 (segment (start 143.5366 107.478) (end 143.5366 104.6492) (width 0.5) (layer "F.Cu") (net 41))
 (segment (start 127.8382 104.5972) (end 127.4068 104.1658) (width 0.5) (layer "F.Cu") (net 41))
 (segment (start 127.4068 104.1658) (end 127.4068 96.9264) (width 0.5) (layer "F.Cu") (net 41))
 (segment (start 143.5366 104.6492) (end 143.4846 104.5972) (width 0.25) (layer "F.Cu") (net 41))
 (segment (start 143.4846 104.5972) (end 127.8382 104.5972) (width 0.5) (layer "F.Cu") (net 41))
 (segment (start 150.0366 107.478) (end 143.5366 107.478) (width 0.5) (layer "F.Cu") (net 41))
 (segment (start 153.2902 103.5812) (end 130.4544 103.5812) (width 0.5) (layer "F.Cu") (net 42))
 (segment (start 130.4544 103.5812) (end 130.5568 103.4788) (width 0.25) (layer "F.Cu") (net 42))
 (segment (start 159.7902 107.478) (end 153.2902 107.478) (width 0.5) (layer "F.Cu") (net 42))
 (segment (start 130.5568 103.4788) (end 130.5568 96.9264) (width 0.5) (layer "F.Cu") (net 42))
 (segment (start 153.2902 107.478) (end 153.2902 103.5812) (width 0.5) (layer "F.Cu") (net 42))
 (segment (start 163.0692 107.478) (end 163.0692 105.1318) (width 0.5) (layer "F.Cu") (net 1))
 (segment (start 133.7068 102.5664) (end 133.7068 96.9264) (width 0.5) (layer "F.Cu") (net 1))
 (segment (start 169.5692 107.478) (end 163.0692 107.478) (width 0.5) (layer "F.Cu") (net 1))
 (segment (start 133.731 102.5906) (end 133.7068 102.5664) (width 0.5) (layer "F.Cu") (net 1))
 (segment (start 163.0692 105.1318) (end 160.528 102.5906) (width 0.5) (layer "F.Cu") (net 1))
 (segment (start 160.528 102.5906) (end 133.731 102.5906) (width 0.5) (layer "F.Cu") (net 1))
 (segment (start 153.9748 115.6208) (end 151.9936 115.6208) (width 0.5) (layer "B.Cu") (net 14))
 (segment (start 168.1734 105.3084) (end 159.0294 105.3084) (width 0.5) (layer "B.Cu") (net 14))
 (segment (start 151.9936 115.6208) (end 151.9936 117.7544) (width 0.5) (layer "B.Cu") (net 14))
 (segment (start 168.1226 100.2284) (end 168.1734 100.2792) (width 0.5) (layer "B.Cu") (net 14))
 (segment (start 156.972 112.6236) (end 153.9748 115.6208) (width 0.5) (layer "B.Cu") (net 14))
 (segment (start 159.0294 105.3084) (end 156.972 107.3658) (width 0.5) (layer "B.Cu") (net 14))
 (segment (start 156.972 107.3658) (end 156.972 112.6236) (width 0.5) (layer "B.Cu") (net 14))
 (segment (start 168.1734 100.2792) (end 168.1734 105.3084) (width 0.5) (layer "B.Cu") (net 14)))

